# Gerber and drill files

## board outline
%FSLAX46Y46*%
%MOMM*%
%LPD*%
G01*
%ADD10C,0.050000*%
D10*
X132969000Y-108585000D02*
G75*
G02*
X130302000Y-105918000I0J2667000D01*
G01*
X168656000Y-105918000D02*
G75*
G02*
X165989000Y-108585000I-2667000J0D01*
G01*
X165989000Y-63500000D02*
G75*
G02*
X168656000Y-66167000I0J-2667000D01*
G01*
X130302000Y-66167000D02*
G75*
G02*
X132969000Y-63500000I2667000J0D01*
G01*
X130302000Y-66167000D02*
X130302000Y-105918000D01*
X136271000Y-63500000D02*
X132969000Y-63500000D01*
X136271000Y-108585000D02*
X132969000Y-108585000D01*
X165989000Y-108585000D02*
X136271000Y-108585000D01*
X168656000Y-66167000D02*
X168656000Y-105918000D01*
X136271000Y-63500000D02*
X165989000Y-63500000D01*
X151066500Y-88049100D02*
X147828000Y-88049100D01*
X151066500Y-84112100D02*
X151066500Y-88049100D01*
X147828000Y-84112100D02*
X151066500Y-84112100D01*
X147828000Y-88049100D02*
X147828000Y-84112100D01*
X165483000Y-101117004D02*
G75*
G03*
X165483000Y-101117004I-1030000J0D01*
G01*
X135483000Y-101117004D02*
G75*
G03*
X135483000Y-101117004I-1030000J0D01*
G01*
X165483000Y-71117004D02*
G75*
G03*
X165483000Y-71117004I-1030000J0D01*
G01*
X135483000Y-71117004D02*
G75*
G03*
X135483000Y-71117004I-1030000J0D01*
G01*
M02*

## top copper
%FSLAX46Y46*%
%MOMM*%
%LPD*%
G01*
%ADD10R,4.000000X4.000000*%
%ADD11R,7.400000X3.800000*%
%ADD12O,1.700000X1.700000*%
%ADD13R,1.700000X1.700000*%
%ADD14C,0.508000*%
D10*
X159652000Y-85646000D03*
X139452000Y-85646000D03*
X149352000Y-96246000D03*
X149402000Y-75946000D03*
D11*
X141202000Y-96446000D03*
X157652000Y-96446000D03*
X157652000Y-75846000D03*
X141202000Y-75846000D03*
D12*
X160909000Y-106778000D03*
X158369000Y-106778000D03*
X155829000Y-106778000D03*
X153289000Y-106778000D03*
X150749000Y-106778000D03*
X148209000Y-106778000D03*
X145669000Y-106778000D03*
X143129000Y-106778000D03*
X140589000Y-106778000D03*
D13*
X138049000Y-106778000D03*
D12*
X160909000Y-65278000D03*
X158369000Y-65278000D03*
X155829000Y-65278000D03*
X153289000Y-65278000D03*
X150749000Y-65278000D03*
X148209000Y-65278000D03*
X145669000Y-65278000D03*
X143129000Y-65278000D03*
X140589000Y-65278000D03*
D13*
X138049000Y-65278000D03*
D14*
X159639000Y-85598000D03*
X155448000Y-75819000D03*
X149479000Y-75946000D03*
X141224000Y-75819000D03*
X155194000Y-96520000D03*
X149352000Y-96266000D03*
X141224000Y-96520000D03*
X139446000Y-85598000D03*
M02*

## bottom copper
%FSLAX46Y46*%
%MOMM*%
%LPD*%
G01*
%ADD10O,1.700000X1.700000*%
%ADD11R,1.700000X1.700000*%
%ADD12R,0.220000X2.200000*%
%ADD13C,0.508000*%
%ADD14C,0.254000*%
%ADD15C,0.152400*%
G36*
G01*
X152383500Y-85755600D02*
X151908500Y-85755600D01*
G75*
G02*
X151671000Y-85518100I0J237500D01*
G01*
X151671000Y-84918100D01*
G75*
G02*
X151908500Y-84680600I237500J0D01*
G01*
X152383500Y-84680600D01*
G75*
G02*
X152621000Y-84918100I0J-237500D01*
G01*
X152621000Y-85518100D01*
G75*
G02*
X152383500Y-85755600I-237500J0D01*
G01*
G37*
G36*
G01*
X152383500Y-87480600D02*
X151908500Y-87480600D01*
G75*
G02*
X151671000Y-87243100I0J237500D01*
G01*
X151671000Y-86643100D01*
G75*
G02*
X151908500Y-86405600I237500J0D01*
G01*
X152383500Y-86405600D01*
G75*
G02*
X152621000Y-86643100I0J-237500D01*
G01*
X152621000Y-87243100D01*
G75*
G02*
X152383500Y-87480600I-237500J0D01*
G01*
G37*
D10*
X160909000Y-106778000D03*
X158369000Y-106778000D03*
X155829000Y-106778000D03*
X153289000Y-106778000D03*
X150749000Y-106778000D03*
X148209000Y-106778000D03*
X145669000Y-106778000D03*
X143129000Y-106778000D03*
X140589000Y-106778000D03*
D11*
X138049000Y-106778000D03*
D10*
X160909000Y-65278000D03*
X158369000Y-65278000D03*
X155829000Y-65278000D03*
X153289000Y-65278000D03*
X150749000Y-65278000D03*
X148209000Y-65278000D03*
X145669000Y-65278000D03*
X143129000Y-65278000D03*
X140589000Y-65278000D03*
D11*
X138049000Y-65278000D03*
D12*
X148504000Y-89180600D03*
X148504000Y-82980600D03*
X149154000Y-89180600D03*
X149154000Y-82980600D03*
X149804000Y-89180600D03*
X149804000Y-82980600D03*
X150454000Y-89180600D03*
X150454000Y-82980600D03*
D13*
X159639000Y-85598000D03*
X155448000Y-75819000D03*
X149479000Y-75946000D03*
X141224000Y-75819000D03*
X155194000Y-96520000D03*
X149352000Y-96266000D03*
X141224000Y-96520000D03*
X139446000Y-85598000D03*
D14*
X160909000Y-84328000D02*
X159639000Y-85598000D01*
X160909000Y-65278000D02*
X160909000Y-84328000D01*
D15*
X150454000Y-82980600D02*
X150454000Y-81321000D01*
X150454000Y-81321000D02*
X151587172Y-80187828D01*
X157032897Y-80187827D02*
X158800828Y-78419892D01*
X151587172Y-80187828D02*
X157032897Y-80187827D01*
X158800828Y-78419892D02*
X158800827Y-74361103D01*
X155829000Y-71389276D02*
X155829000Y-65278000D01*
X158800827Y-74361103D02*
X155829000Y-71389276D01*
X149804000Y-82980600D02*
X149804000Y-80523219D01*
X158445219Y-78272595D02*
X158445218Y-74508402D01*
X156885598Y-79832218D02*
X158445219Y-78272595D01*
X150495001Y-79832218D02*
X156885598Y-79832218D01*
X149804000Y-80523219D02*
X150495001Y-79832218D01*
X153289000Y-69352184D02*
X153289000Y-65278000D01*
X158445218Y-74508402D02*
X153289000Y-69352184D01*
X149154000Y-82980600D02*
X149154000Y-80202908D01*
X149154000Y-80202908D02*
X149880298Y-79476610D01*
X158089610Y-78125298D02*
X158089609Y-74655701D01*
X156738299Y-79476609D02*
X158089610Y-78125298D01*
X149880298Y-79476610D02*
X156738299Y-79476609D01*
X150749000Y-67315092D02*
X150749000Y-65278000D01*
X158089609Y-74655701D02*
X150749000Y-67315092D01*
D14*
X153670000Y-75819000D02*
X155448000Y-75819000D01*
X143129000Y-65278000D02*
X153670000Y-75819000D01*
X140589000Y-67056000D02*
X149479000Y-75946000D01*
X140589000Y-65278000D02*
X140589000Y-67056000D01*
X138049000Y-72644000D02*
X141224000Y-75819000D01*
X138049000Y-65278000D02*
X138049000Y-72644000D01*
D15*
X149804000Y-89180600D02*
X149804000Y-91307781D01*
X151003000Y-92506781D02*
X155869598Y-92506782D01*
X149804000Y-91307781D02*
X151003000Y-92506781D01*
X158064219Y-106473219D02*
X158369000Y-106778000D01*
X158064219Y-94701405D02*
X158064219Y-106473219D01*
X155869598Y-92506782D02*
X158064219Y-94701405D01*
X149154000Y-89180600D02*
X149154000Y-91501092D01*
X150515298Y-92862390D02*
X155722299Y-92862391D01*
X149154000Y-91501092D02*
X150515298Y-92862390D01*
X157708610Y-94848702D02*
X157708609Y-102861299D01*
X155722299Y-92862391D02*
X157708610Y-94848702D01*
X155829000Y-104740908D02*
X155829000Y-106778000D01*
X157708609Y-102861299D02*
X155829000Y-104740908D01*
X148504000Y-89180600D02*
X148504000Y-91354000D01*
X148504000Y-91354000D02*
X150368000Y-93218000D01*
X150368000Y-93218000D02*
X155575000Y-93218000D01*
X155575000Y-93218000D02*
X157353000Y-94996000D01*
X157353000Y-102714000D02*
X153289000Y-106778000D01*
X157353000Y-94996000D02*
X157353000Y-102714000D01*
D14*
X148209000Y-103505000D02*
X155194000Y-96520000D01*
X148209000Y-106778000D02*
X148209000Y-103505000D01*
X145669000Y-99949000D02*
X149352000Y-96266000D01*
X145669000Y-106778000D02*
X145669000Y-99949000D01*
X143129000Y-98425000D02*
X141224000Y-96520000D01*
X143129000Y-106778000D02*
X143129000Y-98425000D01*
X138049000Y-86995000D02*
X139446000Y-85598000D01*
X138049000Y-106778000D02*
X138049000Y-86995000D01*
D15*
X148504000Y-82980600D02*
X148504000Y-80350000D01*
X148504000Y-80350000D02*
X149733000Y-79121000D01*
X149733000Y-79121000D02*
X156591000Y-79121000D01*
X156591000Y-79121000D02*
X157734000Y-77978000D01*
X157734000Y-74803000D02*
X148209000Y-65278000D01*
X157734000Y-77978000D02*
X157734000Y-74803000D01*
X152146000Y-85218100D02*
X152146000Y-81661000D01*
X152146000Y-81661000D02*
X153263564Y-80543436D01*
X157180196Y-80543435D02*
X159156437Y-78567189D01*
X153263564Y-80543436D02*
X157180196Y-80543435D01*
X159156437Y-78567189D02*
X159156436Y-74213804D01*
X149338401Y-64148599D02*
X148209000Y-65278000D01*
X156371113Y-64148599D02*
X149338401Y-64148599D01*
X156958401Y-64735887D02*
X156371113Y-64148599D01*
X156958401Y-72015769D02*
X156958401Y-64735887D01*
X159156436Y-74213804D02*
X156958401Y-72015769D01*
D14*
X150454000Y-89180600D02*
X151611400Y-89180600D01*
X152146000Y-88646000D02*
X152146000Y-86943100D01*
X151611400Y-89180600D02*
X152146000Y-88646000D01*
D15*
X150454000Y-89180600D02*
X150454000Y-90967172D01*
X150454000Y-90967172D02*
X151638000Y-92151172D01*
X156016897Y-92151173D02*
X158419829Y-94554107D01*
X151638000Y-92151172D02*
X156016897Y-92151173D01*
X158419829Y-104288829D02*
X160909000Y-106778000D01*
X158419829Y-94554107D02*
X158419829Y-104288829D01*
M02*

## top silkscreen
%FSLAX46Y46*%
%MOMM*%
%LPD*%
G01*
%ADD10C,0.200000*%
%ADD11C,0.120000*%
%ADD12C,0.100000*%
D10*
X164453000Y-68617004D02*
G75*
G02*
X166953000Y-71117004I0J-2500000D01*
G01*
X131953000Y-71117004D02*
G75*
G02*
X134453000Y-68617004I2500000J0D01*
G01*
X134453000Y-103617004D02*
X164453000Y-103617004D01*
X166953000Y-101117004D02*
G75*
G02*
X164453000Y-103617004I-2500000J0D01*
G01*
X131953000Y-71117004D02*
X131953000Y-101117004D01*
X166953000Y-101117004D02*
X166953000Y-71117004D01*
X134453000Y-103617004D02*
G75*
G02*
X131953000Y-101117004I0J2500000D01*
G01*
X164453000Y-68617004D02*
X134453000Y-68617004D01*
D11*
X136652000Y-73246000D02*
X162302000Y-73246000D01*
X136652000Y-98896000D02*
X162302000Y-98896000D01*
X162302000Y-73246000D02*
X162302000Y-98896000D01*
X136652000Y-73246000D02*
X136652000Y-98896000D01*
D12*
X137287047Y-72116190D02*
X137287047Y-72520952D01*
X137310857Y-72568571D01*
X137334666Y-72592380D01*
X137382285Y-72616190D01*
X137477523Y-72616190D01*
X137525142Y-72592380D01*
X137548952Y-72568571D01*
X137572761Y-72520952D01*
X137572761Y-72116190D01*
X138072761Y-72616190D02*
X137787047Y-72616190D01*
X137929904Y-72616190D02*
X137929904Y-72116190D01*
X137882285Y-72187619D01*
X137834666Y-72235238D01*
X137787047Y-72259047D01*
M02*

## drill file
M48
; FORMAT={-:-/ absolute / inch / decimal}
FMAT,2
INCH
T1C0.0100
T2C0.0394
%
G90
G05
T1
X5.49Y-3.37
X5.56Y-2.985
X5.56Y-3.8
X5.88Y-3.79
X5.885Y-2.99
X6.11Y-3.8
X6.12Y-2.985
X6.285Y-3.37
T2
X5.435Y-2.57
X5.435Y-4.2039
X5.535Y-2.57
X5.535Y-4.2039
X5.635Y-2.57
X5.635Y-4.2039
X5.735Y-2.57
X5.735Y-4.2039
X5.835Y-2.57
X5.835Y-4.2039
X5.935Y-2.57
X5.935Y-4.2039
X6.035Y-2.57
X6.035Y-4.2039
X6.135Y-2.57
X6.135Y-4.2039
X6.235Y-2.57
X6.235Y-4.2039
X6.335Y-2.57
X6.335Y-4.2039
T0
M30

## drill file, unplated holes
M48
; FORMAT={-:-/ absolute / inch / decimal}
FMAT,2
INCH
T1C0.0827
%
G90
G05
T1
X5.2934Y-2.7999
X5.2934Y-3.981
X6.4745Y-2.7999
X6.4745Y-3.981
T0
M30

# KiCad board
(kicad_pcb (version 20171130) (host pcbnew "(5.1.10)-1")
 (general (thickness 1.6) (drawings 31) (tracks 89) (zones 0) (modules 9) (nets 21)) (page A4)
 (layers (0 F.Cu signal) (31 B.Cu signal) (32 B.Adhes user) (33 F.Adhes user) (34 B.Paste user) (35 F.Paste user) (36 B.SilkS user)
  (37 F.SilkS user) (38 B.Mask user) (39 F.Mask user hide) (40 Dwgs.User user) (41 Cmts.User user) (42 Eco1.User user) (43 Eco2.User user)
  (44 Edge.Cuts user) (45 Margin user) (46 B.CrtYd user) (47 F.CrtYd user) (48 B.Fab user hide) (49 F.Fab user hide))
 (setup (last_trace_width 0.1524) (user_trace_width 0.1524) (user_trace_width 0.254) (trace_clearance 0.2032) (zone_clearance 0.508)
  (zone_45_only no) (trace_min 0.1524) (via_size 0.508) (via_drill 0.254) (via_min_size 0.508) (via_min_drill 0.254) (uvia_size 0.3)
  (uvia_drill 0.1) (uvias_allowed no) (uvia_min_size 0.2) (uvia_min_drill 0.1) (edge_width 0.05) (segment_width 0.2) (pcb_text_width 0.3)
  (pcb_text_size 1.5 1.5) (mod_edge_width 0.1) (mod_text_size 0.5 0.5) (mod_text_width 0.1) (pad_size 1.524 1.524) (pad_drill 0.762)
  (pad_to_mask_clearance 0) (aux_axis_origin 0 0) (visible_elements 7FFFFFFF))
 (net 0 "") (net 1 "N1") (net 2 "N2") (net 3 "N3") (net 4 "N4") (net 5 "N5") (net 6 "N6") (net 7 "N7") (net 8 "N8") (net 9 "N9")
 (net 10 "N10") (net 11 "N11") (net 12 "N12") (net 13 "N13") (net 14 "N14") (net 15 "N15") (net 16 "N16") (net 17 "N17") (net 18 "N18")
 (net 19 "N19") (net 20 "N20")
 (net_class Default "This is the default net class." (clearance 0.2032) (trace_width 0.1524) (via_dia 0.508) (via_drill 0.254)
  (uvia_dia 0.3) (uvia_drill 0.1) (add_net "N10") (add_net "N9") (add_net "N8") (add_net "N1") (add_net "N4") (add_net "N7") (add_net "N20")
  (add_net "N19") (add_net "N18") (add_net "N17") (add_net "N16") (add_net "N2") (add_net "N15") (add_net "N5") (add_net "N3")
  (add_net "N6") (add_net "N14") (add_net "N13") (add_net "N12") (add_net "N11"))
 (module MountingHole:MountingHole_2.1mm (layer F.Cu) (at 164.453 101.117004)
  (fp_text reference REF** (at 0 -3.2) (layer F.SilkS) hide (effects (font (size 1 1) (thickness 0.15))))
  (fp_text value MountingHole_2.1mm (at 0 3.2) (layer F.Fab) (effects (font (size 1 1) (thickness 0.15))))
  (pad "" np_thru_hole circle (at 0 0) (size 2.1 2.1) (drill 2.1) (layers *.Cu *.Mask)))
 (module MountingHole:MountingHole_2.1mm (layer F.Cu) (at 164.453 71.117004)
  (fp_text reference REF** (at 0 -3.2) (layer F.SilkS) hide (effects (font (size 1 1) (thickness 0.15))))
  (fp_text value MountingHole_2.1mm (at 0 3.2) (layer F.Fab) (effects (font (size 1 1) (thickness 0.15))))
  (pad "" np_thru_hole circle (at 0 0) (size 2.1 2.1) (drill 2.1) (layers *.Cu *.Mask)))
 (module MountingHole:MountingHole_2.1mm (layer F.Cu) (at 134.453 101.117004)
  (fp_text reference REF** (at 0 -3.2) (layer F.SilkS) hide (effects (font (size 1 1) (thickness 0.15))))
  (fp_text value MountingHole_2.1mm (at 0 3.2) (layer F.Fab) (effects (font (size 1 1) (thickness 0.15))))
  (pad "" np_thru_hole circle (at 0 0) (size 2.1 2.1) (drill 2.1) (layers *.Cu *.Mask)))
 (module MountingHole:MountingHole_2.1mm (layer F.Cu) (at 134.453 71.117004)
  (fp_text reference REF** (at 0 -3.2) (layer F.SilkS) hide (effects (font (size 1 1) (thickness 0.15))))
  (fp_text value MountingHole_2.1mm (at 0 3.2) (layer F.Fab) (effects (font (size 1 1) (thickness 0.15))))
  (pad "" np_thru_hole circle (at 0 0) (size 2.1 2.1) (drill 2.1) (layers *.Cu *.Mask)))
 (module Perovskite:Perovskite (layer F.Cu) (at 136.652 73.246)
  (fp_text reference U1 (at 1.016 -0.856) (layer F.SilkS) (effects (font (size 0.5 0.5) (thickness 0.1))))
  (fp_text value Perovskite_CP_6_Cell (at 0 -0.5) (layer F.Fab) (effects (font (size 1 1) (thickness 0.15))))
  (fp_line (start 0 0) (end 25.65 0) (layer F.SilkS) (width 0.12))
  (fp_line (start 0 25.65) (end 25.65 25.65) (layer F.SilkS) (width 0.12))
  (fp_line (start 25.65 0) (end 25.65 25.65) (layer F.SilkS) (width 0.12))
  (fp_line (start 0 0) (end 0 25.65) (layer F.SilkS) (width 0.12))
  (pad 8 smd rect (at 23 12.4) (size 4 4) (layers F.Cu F.Paste F.Mask) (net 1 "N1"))
  (pad 7 smd rect (at 2.8 12.4) (size 4 4) (layers F.Cu F.Paste F.Mask) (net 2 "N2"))
  (pad 5 smd rect (at 12.7 23) (size 4 4) (layers F.Cu F.Paste F.Mask) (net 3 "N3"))
  (pad 2 smd rect (at 12.75 2.7) (size 4 4) (layers F.Cu F.Paste F.Mask) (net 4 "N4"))
  (pad 6 smd rect (at 4.55 23.2) (size 7.4 3.8) (layers F.Cu F.Paste F.Mask) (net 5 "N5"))
  (pad 4 smd rect (at 21 23.2) (size 7.4 3.8) (layers F.Cu F.Paste F.Mask) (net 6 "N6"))
  (pad 3 smd rect (at 21 2.6) (size 7.4 3.8) (layers F.Cu F.Paste F.Mask) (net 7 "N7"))
  (pad 1 smd rect (at 4.55 2.6) (size 7.4 3.8) (layers F.Cu F.Paste F.Mask) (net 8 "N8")))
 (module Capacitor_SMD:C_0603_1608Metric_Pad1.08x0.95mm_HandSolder (layer B.Cu) (at 152.146 86.0806 90)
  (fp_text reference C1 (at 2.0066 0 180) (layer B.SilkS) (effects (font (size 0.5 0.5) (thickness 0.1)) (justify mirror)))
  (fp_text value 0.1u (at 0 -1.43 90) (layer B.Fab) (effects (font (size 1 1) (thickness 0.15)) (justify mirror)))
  (pad 2 smd roundrect (at 0.8625 0 90) (size 1.075 0.95) (layers B.Cu B.Paste B.Mask) (roundrect_rratio 0.25) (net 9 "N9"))
  (pad 1 smd roundrect (at -0.8625 0 90) (size 1.075 0.95) (layers B.Cu B.Paste B.Mask) (roundrect_rratio 0.25) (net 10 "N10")))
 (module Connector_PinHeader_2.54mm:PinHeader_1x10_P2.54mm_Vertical (layer B.Cu) (at 138.049 106.778 270)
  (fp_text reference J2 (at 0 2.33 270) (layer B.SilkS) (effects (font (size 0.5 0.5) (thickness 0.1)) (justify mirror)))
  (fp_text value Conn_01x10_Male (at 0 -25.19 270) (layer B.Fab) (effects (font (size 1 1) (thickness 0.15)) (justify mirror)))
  (pad 10 thru_hole oval (at 0 -22.86 270) (size 1.7 1.7) (drill 1) (layers *.Cu *.Mask) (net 10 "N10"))
  (pad 9 thru_hole oval (at 0 -20.32 270) (size 1.7 1.7) (drill 1) (layers *.Cu *.Mask) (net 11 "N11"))
  (pad 8 thru_hole oval (at 0 -17.78 270) (size 1.7 1.7) (drill 1) (layers *.Cu *.Mask) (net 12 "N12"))
  (pad 7 thru_hole oval (at 0 -15.24 270) (size 1.7 1.7) (drill 1) (layers *.Cu *.Mask) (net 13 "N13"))
  (pad 6 thru_hole oval (at 0 -12.7 270) (size 1.7 1.7) (drill 1) (layers *.Cu *.Mask) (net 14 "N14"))
  (pad 5 thru_hole oval (at 0 -10.16 270) (size 1.7 1.7) (drill 1) (layers *.Cu *.Mask) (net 6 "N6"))
  (pad 4 thru_hole oval (at 0 -7.62 270) (size 1.7 1.7) (drill 1) (layers *.Cu *.Mask) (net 3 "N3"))
  (pad 3 thru_hole oval (at 0 -5.08 270) (size 1.7 1.7) (drill 1) (layers *.Cu *.Mask) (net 5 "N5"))
  (pad 2 thru_hole oval (at 0 -2.54 270) (size 1.7 1.7) (drill 1) (layers *.Cu *.Mask) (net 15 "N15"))
  (pad 1 thru_hole rect (at 0 0 270) (size 1.7 1.7) (drill 1) (layers *.Cu *.Mask) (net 2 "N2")))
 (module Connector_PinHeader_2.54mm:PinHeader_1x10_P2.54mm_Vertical (layer B.Cu) (at 138.049 65.278 270)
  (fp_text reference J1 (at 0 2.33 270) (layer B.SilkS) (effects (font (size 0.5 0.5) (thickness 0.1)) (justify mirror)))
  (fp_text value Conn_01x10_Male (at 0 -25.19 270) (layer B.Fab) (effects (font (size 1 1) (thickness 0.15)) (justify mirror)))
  (pad 10 thru_hole oval (at 0 -22.86 270) (size 1.7 1.7) (drill 1) (layers *.Cu *.Mask) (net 1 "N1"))
  (pad 9 thru_hole oval (at 0 -20.32 270) (size 1.7 1.7) (drill 1) (layers *.Cu *.Mask) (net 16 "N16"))
  (pad 8 thru_hole oval (at 0 -17.78 270) (size 1.7 1.7) (drill 1) (layers *.Cu *.Mask) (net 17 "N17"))
  (pad 7 thru_hole oval (at 0 -15.24 270) (size 1.7 1.7) (drill 1) (layers *.Cu *.Mask) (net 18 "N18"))
  (pad 6 thru_hole oval (at 0 -12.7 270) (size 1.7 1.7) (drill 1) (layers *.Cu *.Mask) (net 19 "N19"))
  (pad 5 thru_hole oval (at 0 -10.16 270) (size 1.7 1.7) (drill 1) (layers *.Cu *.Mask) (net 9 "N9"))
  (pad 4 thru_hole oval (at 0 -7.62 270) (size 1.7 1.7) (drill 1) (layers *.Cu *.Mask) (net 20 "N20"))
  (pad 3 thru_hole oval (at 0 -5.08 270) (size 1.7 1.7) (drill 1) (layers *.Cu *.Mask) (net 7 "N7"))
  (pad 2 thru_hole oval (at 0 -2.54 270) (size 1.7 1.7) (drill 1) (layers *.Cu *.Mask) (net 4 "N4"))
  (pad 1 thru_hole rect (at 0 0 270) (size 1.7 1.7) (drill 1) (layers *.Cu *.Mask) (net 8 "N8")))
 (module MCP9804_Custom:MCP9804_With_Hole (layer B.Cu) (at 149.479 86.0806 90)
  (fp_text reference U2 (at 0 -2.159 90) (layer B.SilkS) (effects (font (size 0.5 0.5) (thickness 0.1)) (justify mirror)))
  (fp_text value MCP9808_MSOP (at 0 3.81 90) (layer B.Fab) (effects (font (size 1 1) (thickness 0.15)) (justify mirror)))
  (pad 5 smd rect (at -3.1 -0.975 180) (size 0.22 2.2) (layers B.Cu B.Paste B.Mask) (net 13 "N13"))
  (pad 4 smd rect (at 3.1 -0.975 180) (size 0.22 2.2) (layers B.Cu B.Paste B.Mask) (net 9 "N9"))
  (pad 6 smd rect (at -3.1 -0.325 180) (size 0.22 2.2) (layers B.Cu B.Paste B.Mask) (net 12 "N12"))
  (pad 3 smd rect (at 3.1 -0.325 180) (size 0.22 2.2) (layers B.Cu B.Paste B.Mask) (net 19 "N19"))
  (pad 7 smd rect (at -3.1 0.325 180) (size 0.22 2.2) (layers B.Cu B.Paste B.Mask) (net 11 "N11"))
  (pad 2 smd rect (at 3.1 0.325 180) (size 0.22 2.2) (layers B.Cu B.Paste B.Mask) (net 18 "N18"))
  (pad 8 smd rect (at -3.1 0.975 180) (size 0.22 2.2) (layers B.Cu B.Paste B.Mask) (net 10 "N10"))
  (pad 1 smd rect (at 3.1 0.975 180) (size 0.22 2.2) (layers B.Cu B.Paste B.Mask) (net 17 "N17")))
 (gr_arc (start 132.969 105.918) (end 130.302 105.918) (angle -90) (layer Edge.Cuts) (width 0.05))
 (gr_arc (start 165.989 105.918) (end 165.989 108.585) (angle -90) (layer Edge.Cuts) (width 0.05))
 (gr_arc (start 165.989 66.167) (end 168.656 66.167) (angle -90) (layer Edge.Cuts) (width 0.05))
 (gr_arc (start 132.969 66.167) (end 132.969 63.5) (angle -90) (layer Edge.Cuts) (width 0.05))
 (gr_line (start 130.302 66.167) (end 130.302 105.918) (layer Edge.Cuts) (width 0.05))
 (gr_line (start 136.271 63.5) (end 132.969 63.5) (layer Edge.Cuts) (width 0.05))
 (gr_line (start 136.271 108.585) (end 132.969 108.585) (layer Edge.Cuts) (width 0.05))
 (gr_line (start 165.989 108.585) (end 136.271 108.585) (layer Edge.Cuts) (width 0.05))
 (gr_line (start 168.656 66.167) (end 168.656 105.918) (layer Edge.Cuts) (width 0.05))
 (gr_line (start 136.271 63.5) (end 165.989 63.5) (layer Edge.Cuts) (width 0.05))
 (gr_line (start 151.0665 88.0491) (end 147.828 88.0491) (layer Edge.Cuts) (width 0.05))
 (gr_line (start 151.0665 84.1121) (end 151.0665 88.0491) (layer Edge.Cuts) (width 0.05))
 (gr_line (start 147.828 84.1121) (end 151.0665 84.1121) (layer Edge.Cuts) (width 0.05))
 (gr_line (start 147.828 88.0491) (end 147.828 84.1121) (layer Edge.Cuts) (width 0.05))
 (gr_arc (start 164.453 71.117004) (end 166.953 71.117004) (angle -90) (layer F.SilkS) (width 0.2))
 (gr_circle (center 164.453 101.117004) (end 165.483 101.117004) (layer Edge.Cuts) (width 0.05))
 (gr_arc (start 134.453 71.117004) (end 134.453 68.617004) (angle -90) (layer F.SilkS) (width 0.2))
 (gr_line (start 134.453 103.617004) (end 164.453 103.617004) (layer F.SilkS) (width 0.2))
 (gr_arc (start 164.453 101.117004) (end 164.453 103.617004) (angle -90) (layer F.SilkS) (width 0.2))
 (gr_line (start 131.953 71.117004) (end 131.953 101.117004) (layer F.SilkS) (width 0.2))
 (gr_line (start 166.953 101.117004) (end 166.953 71.117004) (layer F.SilkS) (width 0.2))
 (gr_circle (center 134.453 101.117004) (end 135.483 101.117004) (layer Edge.Cuts) (width 0.05))
 (gr_arc (start 134.453 101.117004) (end 131.953 101.117004) (angle -90) (layer F.SilkS) (width 0.2))
 (gr_circle (center 164.453 71.117004) (end 165.483 71.117004) (layer Edge.Cuts) (width 0.05))
 (gr_circle (center 134.453 71.117004) (end 135.483 71.117004) (layer Edge.Cuts) (width 0.05))
 (gr_line (start 164.453 68.617004) (end 134.453 68.617004) (layer F.SilkS) (width 0.2))
 (via (at 159.639 85.598) (size 0.508) (drill 0.254) (layers F.Cu B.Cu) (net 1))
 (segment (start 160.909 84.328) (end 159.639 85.598) (width 0.254) (layer B.Cu) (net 1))
 (segment (start 160.909 65.278) (end 160.909 84.328) (width 0.254) (layer B.Cu) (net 1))
 (segment (start 150.454 82.9806) (end 150.454 81.321) (width 0.1524) (layer B.Cu) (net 17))
 (segment (start 150.454 81.321) (end 151.587172 80.187828) (width 0.1524) (layer B.Cu) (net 17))
 (segment (start 157.032897 80.187827) (end 158.800828 78.419892) (width 0.1524) (layer B.Cu) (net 17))
 (segment (start 151.587172 80.187828) (end 157.032897 80.187827) (width 0.1524) (layer B.Cu) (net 17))
 (segment (start 158.800828 78.419892) (end 158.800827 74.361103) (width 0.1524) (layer B.Cu) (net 17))
 (segment (start 155.829 71.389276) (end 155.829 65.278) (width 0.1524) (layer B.Cu) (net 17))
 (segment (start 158.800827 74.361103) (end 155.829 71.389276) (width 0.1524) (layer B.Cu) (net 17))
 (segment (start 149.804 82.9806) (end 149.804 80.523219) (width 0.1524) (layer B.Cu) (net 18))
 (segment (start 158.445219 78.272595) (end 158.445218 74.508402) (width 0.1524) (layer B.Cu) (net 18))
 (segment (start 156.885598 79.832218) (end 158.445219 78.272595) (width 0.1524) (layer B.Cu) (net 18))
 (segment (start 150.495001 79.832218) (end 156.885598 79.832218) (width 0.1524) (layer B.Cu) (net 18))
 (segment (start 149.804 80.523219) (end 150.495001 79.832218) (width 0.1524) (layer B.Cu) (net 18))
 (segment (start 153.289 69.352184) (end 153.289 65.278) (width 0.1524) (layer B.Cu) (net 18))
 (segment (start 158.445218 74.508402) (end 153.289 69.352184) (width 0.1524) (layer B.Cu) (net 18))
 (segment (start 149.154 82.9806) (end 149.154 80.202908) (width 0.1524) (layer B.Cu) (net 19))
 (segment (start 149.154 80.202908) (end 149.880298 79.47661) (width 0.1524) (layer B.Cu) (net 19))
 (segment (start 158.08961 78.125298) (end 158.089609 74.655701) (width 0.1524) (layer B.Cu) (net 19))
 (segment (start 156.738299 79.476609) (end 158.08961 78.125298) (width 0.1524) (layer B.Cu) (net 19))
 (segment (start 149.880298 79.47661) (end 156.738299 79.476609) (width 0.1524) (layer B.Cu) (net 19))
 (segment (start 150.749 67.315092) (end 150.749 65.278) (width 0.1524) (layer B.Cu) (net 19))
 (segment (start 158.089609 74.655701) (end 150.749 67.315092) (width 0.1524) (layer B.Cu) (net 19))
 (via (at 155.448 75.819) (size 0.508) (drill 0.254) (layers F.Cu B.Cu) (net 7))
 (segment (start 153.67 75.819) (end 155.448 75.819) (width 0.254) (layer B.Cu) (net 7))
 (segment (start 143.129 65.278) (end 153.67 75.819) (width 0.254) (layer B.Cu) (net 7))
 (via (at 149.479 75.946) (size 0.508) (drill 0.254) (layers F.Cu B.Cu) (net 4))
 (segment (start 140.589 67.056) (end 149.479 75.946) (width 0.254) (layer B.Cu) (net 4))
 (segment (start 140.589 65.278) (end 140.589 67.056) (width 0.254) (layer B.Cu) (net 4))
 (via (at 141.224 75.819) (size 0.508) (drill 0.254) (layers F.Cu B.Cu) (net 8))
 (segment (start 138.049 72.644) (end 141.224 75.819) (width 0.254) (layer B.Cu) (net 8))
 (segment (start 138.049 65.278) (end 138.049 72.644) (width 0.254) (layer B.Cu) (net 8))
 (segment (start 149.804 89.1806) (end 149.804 91.307781) (width 0.1524) (layer B.Cu) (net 11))
 (segment (start 151.003 92.506781) (end 155.869598 92.506782) (width 0.1524) (layer B.Cu) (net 11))
 (segment (start 149.804 91.307781) (end 151.003 92.506781) (width 0.1524) (layer B.Cu) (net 11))
 (segment (start 158.064219 106.473219) (end 158.369 106.778) (width 0.1524) (layer B.Cu) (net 11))
 (segment (start 158.064219 94.701405) (end 158.064219 106.473219) (width 0.1524) (layer B.Cu) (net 11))
 (segment (start 155.869598 92.506782) (end 158.064219 94.701405) (width 0.1524) (layer B.Cu) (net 11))
 (segment (start 149.154 89.1806) (end 149.154 91.501092) (width 0.1524) (layer B.Cu) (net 12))
 (segment (start 150.515298 92.86239) (end 155.722299 92.862391) (width 0.1524) (layer B.Cu) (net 12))
 (segment (start 149.154 91.501092) (end 150.515298 92.86239) (width 0.1524) (layer B.Cu) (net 12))
 (segment (start 157.70861 94.848702) (end 157.708609 102.861299) (width 0.1524) (layer B.Cu) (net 12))
 (segment (start 155.722299 92.862391) (end 157.70861 94.848702) (width 0.1524) (layer B.Cu) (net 12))
 (segment (start 155.829 104.740908) (end 155.829 106.778) (width 0.1524) (layer B.Cu) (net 12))
 (segment (start 157.708609 102.861299) (end 155.829 104.740908) (width 0.1524) (layer B.Cu) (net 12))
 (segment (start 148.504 89.1806) (end 148.504 91.354) (width 0.1524) (layer B.Cu) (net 13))
 (segment (start 148.504 91.354) (end 150.368 93.218) (width 0.1524) (layer B.Cu) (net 13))
 (segment (start 150.368 93.218) (end 155.575 93.218) (width 0.1524) (layer B.Cu) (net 13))
 (segment (start 155.575 93.218) (end 157.353 94.996) (width 0.1524) (layer B.Cu) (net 13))
 (segment (start 157.353 102.714) (end 153.289 106.778) (width 0.1524) (layer B.Cu) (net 13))
 (segment (start 157.353 94.996) (end 157.353 102.714) (width 0.1524) (layer B.Cu) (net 13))
 (via (at 155.194 96.52) (size 0.508) (drill 0.254) (layers F.Cu B.Cu) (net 6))
 (segment (start 148.209 103.505) (end 155.194 96.52) (width 0.254) (layer B.Cu) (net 6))
 (segment (start 148.209 106.778) (end 148.209 103.505) (width 0.254) (layer B.Cu) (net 6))
 (via (at 149.352 96.266) (size 0.508) (drill 0.254) (layers F.Cu B.Cu) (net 3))
 (segment (start 145.669 99.949) (end 149.352 96.266) (width 0.254) (layer B.Cu) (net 3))
 (segment (start 145.669 106.778) (end 145.669 99.949) (width 0.254) (layer B.Cu) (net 3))
 (via (at 141.224 96.52) (size 0.508) (drill 0.254) (layers F.Cu B.Cu) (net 5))
 (segment (start 143.129 98.425) (end 141.224 96.52) (width 0.254) (layer B.Cu) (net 5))
 (segment (start 143.129 106.778) (end 143.129 98.425) (width 0.254) (layer B.Cu) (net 5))
 (via (at 139.446 85.598) (size 0.508) (drill 0.254) (layers F.Cu B.Cu) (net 2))
 (segment (start 138.049 86.995) (end 139.446 85.598) (width 0.254) (layer B.Cu) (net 2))
 (segment (start 138.049 106.778) (end 138.049 86.995) (width 0.254) (layer B.Cu) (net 2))
 (segment (start 148.504 82.9806) (end 148.504 80.35) (width 0.1524) (layer B.Cu) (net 9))
 (segment (start 148.504 80.35) (end 149.733 79.121) (width 0.1524) (layer B.Cu) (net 9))
 (segment (start 149.733 79.121) (end 156.591 79.121) (width 0.1524) (layer B.Cu) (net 9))
 (segment (start 156.591 79.121) (end 157.734 77.978) (width 0.1524) (layer B.Cu) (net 9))
 (segment (start 157.734 74.803) (end 148.209 65.278) (width 0.1524) (layer B.Cu) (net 9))
 (segment (start 157.734 77.978) (end 157.734 74.803) (width 0.1524) (layer B.Cu) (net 9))
 (segment (start 152.146 85.2181) (end 152.146 81.661) (width 0.1524) (layer B.Cu) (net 9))
 (segment (start 152.146 81.661) (end 153.263564 80.543436) (width 0.1524) (layer B.Cu) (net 9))
 (segment (start 157.180196 80.543435) (end 159.156437 78.567189) (width 0.1524) (layer B.Cu) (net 9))
 (segment (start 153.263564 80.543436) (end 157.180196 80.543435) (width 0.1524) (layer B.Cu) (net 9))
 (segment (start 159.156437 78.567189) (end 159.156436 74.213804) (width 0.1524) (layer B.Cu) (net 9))
 (segment (start 149.338401 64.148599) (end 148.209 65.278) (width 0.1524) (layer B.Cu) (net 9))
 (segment (start 156.371113 64.148599) (end 149.338401 64.148599) (width 0.1524) (layer B.Cu) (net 9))
 (segment (start 156.958401 64.735887) (end 156.371113 64.148599) (width 0.1524) (layer B.Cu) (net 9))
 (segment (start 156.958401 72.015769) (end 156.958401 64.735887) (width 0.1524) (layer B.Cu) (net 9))
 (segment (start 159.156436 74.213804) (end 156.958401 72.015769) (width 0.1524) (layer B.Cu) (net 9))
 (segment (start 150.454 89.1806) (end 151.6114 89.1806) (width 0.254) (layer B.Cu) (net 10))
 (segment (start 152.146 88.646) (end 152.146 86.9431) (width 0.254) (layer B.Cu) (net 10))
 (segment (start 151.6114 89.1806) (end 152.146 88.646) (width 0.254) (layer B.Cu) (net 10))
 (segment (start 150.454 89.1806) (end 150.454 90.967172) (width 0.1524) (layer B.Cu) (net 10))
 (segment (start 150.454 90.967172) (end 151.638 92.151172) (width 0.1524) (layer B.Cu) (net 10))
 (segment (start 156.016897 92.151173) (end 158.419829 94.554107) (width 0.1524) (layer B.Cu) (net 10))
 (segment (start 151.638 92.151172) (end 156.016897 92.151173) (width 0.1524) (layer B.Cu) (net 10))
 (segment (start 158.419829 104.288829) (end 160.909 106.778) (width 0.1524) (layer B.Cu) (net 10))
 (segment (start 158.419829 94.554107) (end 158.419829 104.288829) (width 0.1524) (layer B.Cu) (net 10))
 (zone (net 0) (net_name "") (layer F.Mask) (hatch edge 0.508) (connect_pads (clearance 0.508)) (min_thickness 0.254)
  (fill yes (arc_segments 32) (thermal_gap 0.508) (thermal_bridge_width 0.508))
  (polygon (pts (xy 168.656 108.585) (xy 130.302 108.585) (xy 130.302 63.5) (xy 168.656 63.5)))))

